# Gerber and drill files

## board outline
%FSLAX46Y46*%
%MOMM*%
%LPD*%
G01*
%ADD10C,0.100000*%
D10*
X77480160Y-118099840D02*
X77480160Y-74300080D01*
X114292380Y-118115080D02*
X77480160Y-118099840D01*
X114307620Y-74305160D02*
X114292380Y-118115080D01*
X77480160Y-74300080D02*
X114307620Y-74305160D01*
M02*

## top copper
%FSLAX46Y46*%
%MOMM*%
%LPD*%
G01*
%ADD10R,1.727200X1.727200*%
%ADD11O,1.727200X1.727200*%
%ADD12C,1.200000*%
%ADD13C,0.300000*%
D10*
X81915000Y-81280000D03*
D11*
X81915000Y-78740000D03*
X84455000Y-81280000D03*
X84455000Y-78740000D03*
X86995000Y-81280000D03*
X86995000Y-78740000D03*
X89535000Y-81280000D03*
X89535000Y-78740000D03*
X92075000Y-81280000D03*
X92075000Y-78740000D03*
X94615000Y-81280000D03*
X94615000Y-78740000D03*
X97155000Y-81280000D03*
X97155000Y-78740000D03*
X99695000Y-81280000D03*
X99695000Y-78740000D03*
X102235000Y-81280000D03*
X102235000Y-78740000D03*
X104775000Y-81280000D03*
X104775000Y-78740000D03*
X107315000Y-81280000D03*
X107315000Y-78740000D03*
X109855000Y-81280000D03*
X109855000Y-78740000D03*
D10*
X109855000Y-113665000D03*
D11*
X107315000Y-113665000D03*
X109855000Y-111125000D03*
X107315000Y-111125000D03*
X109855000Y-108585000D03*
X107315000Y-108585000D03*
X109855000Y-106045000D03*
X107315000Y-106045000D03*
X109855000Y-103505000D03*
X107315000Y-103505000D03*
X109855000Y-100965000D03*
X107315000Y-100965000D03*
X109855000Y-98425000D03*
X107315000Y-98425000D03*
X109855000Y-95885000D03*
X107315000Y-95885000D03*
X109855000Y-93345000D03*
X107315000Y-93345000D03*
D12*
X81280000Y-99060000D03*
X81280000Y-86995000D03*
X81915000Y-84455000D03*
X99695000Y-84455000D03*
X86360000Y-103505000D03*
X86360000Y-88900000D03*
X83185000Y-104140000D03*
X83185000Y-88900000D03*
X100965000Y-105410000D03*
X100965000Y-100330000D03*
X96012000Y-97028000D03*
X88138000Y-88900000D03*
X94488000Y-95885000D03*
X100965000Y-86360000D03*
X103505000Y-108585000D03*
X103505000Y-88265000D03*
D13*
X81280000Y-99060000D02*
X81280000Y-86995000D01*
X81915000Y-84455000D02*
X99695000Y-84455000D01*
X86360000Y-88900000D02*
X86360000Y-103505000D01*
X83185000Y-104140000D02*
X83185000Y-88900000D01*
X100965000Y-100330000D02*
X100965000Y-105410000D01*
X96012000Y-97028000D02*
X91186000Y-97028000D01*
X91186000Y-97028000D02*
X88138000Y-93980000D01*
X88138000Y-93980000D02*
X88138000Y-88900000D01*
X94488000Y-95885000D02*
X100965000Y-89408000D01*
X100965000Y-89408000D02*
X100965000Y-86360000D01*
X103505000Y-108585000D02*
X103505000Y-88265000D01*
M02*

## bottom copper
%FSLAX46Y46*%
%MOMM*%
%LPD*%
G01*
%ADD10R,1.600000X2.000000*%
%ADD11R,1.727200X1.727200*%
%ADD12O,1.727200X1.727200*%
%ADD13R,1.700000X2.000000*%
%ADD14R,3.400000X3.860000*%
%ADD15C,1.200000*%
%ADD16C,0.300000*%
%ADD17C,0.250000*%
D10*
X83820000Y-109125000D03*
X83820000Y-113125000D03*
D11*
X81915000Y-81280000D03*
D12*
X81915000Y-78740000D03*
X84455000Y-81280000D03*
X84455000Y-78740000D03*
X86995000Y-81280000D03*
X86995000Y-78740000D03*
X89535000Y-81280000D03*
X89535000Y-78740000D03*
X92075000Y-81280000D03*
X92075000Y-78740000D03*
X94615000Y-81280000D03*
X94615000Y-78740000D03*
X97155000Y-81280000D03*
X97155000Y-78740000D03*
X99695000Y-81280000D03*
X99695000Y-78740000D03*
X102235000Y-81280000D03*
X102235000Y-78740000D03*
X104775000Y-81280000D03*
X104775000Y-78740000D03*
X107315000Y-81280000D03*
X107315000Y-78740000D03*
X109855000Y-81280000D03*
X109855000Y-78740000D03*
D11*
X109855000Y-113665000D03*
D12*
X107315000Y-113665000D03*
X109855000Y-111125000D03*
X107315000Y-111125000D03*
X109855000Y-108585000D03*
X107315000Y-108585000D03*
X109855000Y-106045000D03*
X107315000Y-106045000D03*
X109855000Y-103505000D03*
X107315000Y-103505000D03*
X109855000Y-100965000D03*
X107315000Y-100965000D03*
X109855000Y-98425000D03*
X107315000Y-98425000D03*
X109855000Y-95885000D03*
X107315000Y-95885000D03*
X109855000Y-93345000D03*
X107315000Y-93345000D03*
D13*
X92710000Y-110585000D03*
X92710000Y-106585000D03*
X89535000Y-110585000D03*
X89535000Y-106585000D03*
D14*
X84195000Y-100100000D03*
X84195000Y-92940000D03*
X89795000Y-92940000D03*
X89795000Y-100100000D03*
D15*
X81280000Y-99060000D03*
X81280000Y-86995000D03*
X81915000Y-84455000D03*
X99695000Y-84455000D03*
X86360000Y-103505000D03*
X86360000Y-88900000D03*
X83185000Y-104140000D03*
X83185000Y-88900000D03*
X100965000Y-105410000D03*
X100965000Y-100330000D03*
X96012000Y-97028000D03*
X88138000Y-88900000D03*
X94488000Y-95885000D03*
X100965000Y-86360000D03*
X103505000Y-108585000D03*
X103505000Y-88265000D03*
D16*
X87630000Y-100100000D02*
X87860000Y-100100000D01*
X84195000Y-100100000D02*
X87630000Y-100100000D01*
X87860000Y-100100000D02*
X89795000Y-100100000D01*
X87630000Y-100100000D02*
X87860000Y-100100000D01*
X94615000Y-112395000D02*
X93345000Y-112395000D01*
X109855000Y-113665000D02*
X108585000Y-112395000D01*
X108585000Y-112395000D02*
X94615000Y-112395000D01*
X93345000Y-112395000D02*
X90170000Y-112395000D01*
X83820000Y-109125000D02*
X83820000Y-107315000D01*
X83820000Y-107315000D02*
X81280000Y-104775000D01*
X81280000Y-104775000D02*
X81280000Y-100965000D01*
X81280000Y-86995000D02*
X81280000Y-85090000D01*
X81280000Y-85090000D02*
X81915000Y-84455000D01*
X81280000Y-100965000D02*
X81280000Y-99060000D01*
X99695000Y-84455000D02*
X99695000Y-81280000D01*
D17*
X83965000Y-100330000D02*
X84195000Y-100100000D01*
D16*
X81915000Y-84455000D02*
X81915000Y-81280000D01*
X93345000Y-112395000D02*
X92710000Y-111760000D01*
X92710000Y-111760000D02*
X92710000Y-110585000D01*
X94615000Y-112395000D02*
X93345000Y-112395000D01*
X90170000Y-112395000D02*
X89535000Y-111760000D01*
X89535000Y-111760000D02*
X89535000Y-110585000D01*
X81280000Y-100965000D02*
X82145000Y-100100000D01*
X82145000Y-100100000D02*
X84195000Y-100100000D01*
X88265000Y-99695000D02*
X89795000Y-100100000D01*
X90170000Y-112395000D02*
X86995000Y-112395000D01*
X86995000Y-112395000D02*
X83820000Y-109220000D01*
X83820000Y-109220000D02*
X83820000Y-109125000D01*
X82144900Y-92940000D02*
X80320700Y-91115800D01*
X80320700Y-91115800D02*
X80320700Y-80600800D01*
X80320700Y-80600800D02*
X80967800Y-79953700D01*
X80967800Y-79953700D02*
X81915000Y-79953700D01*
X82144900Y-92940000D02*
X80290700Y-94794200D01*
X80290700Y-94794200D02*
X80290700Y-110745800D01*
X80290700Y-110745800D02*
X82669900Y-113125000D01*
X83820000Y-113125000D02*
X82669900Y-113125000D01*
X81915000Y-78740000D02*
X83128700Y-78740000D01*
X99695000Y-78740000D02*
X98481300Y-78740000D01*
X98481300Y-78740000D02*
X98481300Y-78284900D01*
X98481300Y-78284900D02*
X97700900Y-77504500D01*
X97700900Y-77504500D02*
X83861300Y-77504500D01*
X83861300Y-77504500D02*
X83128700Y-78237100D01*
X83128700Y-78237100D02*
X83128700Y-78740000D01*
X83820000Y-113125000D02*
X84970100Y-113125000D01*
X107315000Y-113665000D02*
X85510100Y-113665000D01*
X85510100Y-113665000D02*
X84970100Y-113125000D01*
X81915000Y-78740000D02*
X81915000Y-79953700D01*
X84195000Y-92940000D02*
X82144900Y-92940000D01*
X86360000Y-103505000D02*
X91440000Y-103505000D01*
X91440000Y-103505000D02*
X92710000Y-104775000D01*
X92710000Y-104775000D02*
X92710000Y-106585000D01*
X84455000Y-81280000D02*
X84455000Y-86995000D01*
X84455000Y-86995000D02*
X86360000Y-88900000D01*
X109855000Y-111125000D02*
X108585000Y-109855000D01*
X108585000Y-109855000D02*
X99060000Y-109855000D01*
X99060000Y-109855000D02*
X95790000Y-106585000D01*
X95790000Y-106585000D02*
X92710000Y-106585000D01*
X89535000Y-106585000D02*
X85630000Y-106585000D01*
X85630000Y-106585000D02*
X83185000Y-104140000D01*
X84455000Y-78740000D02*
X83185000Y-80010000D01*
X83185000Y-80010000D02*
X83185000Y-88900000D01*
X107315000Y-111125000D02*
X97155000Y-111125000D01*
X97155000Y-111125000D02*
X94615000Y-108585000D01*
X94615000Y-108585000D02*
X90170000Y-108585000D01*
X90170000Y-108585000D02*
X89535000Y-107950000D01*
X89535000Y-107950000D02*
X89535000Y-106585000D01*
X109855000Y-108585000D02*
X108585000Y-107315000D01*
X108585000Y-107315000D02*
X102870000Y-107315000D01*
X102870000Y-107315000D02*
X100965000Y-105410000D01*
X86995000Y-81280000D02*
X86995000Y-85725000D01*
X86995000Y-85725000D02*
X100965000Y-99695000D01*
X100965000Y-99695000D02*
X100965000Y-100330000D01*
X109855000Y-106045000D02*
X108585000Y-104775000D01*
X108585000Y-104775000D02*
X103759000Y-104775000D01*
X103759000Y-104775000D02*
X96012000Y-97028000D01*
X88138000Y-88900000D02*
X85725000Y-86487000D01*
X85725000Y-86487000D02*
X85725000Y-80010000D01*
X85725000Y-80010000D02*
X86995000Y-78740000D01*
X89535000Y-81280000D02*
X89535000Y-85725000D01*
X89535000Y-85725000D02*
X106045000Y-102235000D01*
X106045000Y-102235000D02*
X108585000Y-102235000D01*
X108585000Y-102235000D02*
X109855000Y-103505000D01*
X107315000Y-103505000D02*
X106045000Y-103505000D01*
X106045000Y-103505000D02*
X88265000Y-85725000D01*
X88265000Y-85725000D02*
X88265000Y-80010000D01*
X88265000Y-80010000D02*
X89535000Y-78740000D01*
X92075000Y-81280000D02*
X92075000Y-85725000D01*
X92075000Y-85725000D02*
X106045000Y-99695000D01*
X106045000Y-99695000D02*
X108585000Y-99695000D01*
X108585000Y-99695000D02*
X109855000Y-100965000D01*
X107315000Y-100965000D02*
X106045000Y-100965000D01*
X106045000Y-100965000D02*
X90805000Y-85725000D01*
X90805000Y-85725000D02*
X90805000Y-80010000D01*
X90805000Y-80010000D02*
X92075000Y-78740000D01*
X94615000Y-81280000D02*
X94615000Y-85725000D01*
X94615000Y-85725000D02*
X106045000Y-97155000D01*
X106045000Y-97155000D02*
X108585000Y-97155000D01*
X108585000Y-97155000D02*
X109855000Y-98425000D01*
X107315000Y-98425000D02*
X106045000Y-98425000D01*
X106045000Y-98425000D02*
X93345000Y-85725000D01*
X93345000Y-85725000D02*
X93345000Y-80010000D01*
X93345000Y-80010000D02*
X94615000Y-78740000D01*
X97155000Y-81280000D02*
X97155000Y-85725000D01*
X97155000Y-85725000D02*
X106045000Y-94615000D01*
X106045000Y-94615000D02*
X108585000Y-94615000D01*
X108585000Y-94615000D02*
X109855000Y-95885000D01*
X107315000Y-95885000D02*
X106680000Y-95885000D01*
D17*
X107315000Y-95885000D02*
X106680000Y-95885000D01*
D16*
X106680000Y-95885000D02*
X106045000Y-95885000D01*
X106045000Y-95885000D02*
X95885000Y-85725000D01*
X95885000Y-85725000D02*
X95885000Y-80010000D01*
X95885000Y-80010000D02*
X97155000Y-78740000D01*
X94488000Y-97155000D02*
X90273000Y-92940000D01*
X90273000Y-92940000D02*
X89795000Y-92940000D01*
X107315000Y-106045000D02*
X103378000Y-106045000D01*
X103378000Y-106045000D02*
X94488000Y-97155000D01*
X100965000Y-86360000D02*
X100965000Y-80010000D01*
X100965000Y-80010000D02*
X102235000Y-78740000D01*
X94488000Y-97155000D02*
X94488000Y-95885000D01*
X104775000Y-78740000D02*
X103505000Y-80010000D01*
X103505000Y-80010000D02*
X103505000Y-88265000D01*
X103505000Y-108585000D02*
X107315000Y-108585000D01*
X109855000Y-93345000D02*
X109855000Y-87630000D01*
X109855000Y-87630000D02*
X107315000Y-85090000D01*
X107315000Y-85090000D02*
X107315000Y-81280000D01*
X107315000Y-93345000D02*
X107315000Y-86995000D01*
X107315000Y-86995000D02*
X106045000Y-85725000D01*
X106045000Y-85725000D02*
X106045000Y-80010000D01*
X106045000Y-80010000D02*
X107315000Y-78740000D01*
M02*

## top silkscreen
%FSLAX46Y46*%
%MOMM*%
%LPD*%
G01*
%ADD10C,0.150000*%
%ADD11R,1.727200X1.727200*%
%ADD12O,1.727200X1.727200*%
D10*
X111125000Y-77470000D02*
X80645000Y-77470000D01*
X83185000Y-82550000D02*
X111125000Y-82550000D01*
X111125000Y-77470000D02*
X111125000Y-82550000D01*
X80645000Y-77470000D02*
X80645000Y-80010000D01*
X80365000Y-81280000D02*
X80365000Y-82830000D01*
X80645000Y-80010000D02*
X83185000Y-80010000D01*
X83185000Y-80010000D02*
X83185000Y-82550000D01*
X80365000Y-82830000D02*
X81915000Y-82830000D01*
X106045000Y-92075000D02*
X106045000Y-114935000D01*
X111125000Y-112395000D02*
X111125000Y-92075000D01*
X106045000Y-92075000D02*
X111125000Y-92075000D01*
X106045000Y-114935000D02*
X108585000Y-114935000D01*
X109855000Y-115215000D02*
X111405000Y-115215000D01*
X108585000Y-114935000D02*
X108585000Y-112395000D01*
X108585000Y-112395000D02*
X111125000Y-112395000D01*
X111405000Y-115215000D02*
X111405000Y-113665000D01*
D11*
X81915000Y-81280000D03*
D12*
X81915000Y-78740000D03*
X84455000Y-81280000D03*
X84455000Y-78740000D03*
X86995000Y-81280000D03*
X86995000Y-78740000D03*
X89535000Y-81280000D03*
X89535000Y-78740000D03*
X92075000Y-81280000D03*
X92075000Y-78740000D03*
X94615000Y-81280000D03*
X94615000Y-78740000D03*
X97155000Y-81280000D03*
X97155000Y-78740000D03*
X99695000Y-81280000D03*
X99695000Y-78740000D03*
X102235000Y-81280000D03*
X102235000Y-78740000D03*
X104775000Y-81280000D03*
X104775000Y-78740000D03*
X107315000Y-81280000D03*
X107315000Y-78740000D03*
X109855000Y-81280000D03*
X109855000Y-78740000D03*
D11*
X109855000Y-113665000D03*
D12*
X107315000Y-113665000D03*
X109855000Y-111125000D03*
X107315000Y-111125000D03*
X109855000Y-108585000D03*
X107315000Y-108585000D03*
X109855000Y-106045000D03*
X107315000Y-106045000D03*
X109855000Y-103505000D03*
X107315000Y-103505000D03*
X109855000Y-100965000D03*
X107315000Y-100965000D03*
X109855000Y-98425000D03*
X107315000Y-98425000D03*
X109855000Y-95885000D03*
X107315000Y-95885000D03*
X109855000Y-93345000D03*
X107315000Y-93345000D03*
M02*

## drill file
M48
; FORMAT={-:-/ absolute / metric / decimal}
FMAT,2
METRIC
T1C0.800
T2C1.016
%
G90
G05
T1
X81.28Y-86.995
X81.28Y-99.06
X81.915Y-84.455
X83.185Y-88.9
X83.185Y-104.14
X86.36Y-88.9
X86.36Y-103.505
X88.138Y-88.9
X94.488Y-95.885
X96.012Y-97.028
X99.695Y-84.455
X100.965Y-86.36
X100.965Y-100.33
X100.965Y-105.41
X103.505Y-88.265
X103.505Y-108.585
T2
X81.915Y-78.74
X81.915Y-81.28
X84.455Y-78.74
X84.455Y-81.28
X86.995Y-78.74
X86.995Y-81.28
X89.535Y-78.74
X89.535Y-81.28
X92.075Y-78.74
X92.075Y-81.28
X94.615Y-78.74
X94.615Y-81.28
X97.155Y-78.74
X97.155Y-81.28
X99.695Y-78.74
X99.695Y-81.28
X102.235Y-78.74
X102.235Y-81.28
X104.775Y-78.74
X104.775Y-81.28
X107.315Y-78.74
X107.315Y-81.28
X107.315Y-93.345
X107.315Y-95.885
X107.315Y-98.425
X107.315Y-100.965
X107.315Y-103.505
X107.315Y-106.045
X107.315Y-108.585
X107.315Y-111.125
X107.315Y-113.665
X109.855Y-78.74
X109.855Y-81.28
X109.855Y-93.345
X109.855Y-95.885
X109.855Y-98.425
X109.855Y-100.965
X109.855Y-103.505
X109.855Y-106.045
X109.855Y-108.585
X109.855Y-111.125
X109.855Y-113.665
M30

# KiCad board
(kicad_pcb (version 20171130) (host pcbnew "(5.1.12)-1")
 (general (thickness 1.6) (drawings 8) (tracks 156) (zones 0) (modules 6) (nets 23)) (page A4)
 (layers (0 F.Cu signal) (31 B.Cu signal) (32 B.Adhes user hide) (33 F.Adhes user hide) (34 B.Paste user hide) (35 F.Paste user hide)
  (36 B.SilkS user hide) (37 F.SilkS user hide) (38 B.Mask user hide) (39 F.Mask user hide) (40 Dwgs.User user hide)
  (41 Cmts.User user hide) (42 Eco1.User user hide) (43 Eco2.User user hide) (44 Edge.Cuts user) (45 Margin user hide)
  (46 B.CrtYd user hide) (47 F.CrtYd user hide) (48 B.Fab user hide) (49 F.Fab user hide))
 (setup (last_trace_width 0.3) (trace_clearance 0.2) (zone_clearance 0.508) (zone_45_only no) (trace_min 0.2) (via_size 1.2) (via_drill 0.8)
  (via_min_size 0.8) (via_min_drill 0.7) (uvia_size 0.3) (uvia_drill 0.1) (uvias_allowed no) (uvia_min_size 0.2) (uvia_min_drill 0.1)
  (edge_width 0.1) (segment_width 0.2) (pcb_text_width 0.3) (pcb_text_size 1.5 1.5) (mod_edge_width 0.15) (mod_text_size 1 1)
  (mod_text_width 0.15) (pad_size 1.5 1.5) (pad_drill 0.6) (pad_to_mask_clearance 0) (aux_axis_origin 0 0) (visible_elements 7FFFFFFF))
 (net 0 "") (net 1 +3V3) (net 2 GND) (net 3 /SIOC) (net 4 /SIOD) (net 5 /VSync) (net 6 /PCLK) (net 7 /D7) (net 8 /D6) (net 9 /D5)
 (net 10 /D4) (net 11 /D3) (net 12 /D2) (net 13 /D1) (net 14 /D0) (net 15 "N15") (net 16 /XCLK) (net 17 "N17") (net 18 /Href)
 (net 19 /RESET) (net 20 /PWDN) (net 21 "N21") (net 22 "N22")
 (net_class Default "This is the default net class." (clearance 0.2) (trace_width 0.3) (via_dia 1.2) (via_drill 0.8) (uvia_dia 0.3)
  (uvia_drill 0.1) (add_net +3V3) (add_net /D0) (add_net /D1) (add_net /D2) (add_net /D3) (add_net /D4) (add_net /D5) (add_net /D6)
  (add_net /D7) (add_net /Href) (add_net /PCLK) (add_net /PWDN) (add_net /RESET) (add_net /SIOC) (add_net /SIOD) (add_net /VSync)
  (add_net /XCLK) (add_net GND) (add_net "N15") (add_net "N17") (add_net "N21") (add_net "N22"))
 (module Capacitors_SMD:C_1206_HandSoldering (layer B.Cu) (at 83.82 111.125 270)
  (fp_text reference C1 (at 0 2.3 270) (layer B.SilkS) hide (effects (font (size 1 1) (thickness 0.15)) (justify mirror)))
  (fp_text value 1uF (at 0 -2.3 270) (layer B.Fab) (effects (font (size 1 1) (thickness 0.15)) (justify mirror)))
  (pad 1 smd rect (at -2 0 270) (size 2 1.6) (layers B.Cu B.Paste B.Mask) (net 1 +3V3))
  (pad 2 smd rect (at 2 0 270) (size 2 1.6) (layers B.Cu B.Paste B.Mask) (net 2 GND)))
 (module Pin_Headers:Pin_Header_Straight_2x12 (layer F.Cu) (at 81.915 81.28 90)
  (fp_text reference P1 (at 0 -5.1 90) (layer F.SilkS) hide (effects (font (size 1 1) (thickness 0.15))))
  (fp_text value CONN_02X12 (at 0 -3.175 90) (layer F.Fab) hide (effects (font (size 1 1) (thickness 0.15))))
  (fp_line (start 3.81 29.21) (end 3.81 -1.27) (layer F.SilkS) (width 0.15))
  (fp_line (start -1.27 1.27) (end -1.27 29.21) (layer F.SilkS) (width 0.15))
  (fp_line (start 3.81 29.21) (end -1.27 29.21) (layer F.SilkS) (width 0.15))
  (fp_line (start 3.81 -1.27) (end 1.27 -1.27) (layer F.SilkS) (width 0.15))
  (fp_line (start 0 -1.55) (end -1.55 -1.55) (layer F.SilkS) (width 0.15))
  (fp_line (start 1.27 -1.27) (end 1.27 1.27) (layer F.SilkS) (width 0.15))
  (fp_line (start 1.27 1.27) (end -1.27 1.27) (layer F.SilkS) (width 0.15))
  (fp_line (start -1.55 -1.55) (end -1.55 0) (layer F.SilkS) (width 0.15))
  (pad 1 thru_hole rect (at 0 0 90) (size 1.7272 1.7272) (drill 1.016) (layers *.Cu *.Mask F.SilkS) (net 1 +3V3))
  (pad 2 thru_hole oval (at 2.54 0 90) (size 1.7272 1.7272) (drill 1.016) (layers *.Cu *.Mask F.SilkS) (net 2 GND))
  (pad 3 thru_hole oval (at 0 2.54 90) (size 1.7272 1.7272) (drill 1.016) (layers *.Cu *.Mask F.SilkS) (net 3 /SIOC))
  (pad 4 thru_hole oval (at 2.54 2.54 90) (size 1.7272 1.7272) (drill 1.016) (layers *.Cu *.Mask F.SilkS) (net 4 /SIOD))
  (pad 5 thru_hole oval (at 0 5.08 90) (size 1.7272 1.7272) (drill 1.016) (layers *.Cu *.Mask F.SilkS) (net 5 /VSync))
  (pad 6 thru_hole oval (at 2.54 5.08 90) (size 1.7272 1.7272) (drill 1.016) (layers *.Cu *.Mask F.SilkS) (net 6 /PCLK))
  (pad 7 thru_hole oval (at 0 7.62 90) (size 1.7272 1.7272) (drill 1.016) (layers *.Cu *.Mask F.SilkS) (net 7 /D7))
  (pad 8 thru_hole oval (at 2.54 7.62 90) (size 1.7272 1.7272) (drill 1.016) (layers *.Cu *.Mask F.SilkS) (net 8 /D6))
  (pad 9 thru_hole oval (at 0 10.16 90) (size 1.7272 1.7272) (drill 1.016) (layers *.Cu *.Mask F.SilkS) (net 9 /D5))
  (pad 10 thru_hole oval (at 2.54 10.16 90) (size 1.7272 1.7272) (drill 1.016) (layers *.Cu *.Mask F.SilkS) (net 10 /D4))
  (pad 11 thru_hole oval (at 0 12.7 90) (size 1.7272 1.7272) (drill 1.016) (layers *.Cu *.Mask F.SilkS) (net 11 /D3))
  (pad 12 thru_hole oval (at 2.54 12.7 90) (size 1.7272 1.7272) (drill 1.016) (layers *.Cu *.Mask F.SilkS) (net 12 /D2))
  (pad 13 thru_hole oval (at 0 15.24 90) (size 1.7272 1.7272) (drill 1.016) (layers *.Cu *.Mask F.SilkS) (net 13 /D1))
  (pad 14 thru_hole oval (at 2.54 15.24 90) (size 1.7272 1.7272) (drill 1.016) (layers *.Cu *.Mask F.SilkS) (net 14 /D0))
  (pad 15 thru_hole oval (at 0 17.78 90) (size 1.7272 1.7272) (drill 1.016) (layers *.Cu *.Mask F.SilkS) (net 1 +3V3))
  (pad 16 thru_hole oval (at 2.54 17.78 90) (size 1.7272 1.7272) (drill 1.016) (layers *.Cu *.Mask F.SilkS) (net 2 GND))
  (pad 17 thru_hole oval (at 0 20.32 90) (size 1.7272 1.7272) (drill 1.016) (layers *.Cu *.Mask F.SilkS) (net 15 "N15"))
  (pad 18 thru_hole oval (at 2.54 20.32 90) (size 1.7272 1.7272) (drill 1.016) (layers *.Cu *.Mask F.SilkS) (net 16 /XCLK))
  (pad 19 thru_hole oval (at 0 22.86 90) (size 1.7272 1.7272) (drill 1.016) (layers *.Cu *.Mask F.SilkS) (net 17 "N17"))
  (pad 20 thru_hole oval (at 2.54 22.86 90) (size 1.7272 1.7272) (drill 1.016) (layers *.Cu *.Mask F.SilkS) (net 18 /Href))
  (pad 21 thru_hole oval (at 0 25.4 90) (size 1.7272 1.7272) (drill 1.016) (layers *.Cu *.Mask F.SilkS) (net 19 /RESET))
  (pad 22 thru_hole oval (at 2.54 25.4 90) (size 1.7272 1.7272) (drill 1.016) (layers *.Cu *.Mask F.SilkS) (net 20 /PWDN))
  (pad 23 thru_hole oval (at 0 27.94 90) (size 1.7272 1.7272) (drill 1.016) (layers *.Cu *.Mask F.SilkS) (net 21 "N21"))
  (pad 24 thru_hole oval (at 2.54 27.94 90) (size 1.7272 1.7272) (drill 1.016) (layers *.Cu *.Mask F.SilkS) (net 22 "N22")))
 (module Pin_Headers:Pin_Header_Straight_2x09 (layer F.Cu) (at 109.855 113.665 180)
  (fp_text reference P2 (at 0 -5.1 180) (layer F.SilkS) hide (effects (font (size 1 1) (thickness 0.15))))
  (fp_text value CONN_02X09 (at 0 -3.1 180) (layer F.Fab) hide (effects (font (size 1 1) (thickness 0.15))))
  (fp_line (start 3.81 21.59) (end 3.81 -1.27) (layer F.SilkS) (width 0.15))
  (fp_line (start -1.27 1.27) (end -1.27 21.59) (layer F.SilkS) (width 0.15))
  (fp_line (start 3.81 21.59) (end -1.27 21.59) (layer F.SilkS) (width 0.15))
  (fp_line (start 3.81 -1.27) (end 1.27 -1.27) (layer F.SilkS) (width 0.15))
  (fp_line (start 0 -1.55) (end -1.55 -1.55) (layer F.SilkS) (width 0.15))
  (fp_line (start 1.27 -1.27) (end 1.27 1.27) (layer F.SilkS) (width 0.15))
  (fp_line (start 1.27 1.27) (end -1.27 1.27) (layer F.SilkS) (width 0.15))
  (fp_line (start -1.55 -1.55) (end -1.55 0) (layer F.SilkS) (width 0.15))
  (pad 1 thru_hole rect (at 0 0 180) (size 1.7272 1.7272) (drill 1.016) (layers *.Cu *.Mask F.SilkS) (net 1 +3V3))
  (pad 2 thru_hole oval (at 2.54 0 180) (size 1.7272 1.7272) (drill 1.016) (layers *.Cu *.Mask F.SilkS) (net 2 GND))
  (pad 3 thru_hole oval (at 0 2.54 180) (size 1.7272 1.7272) (drill 1.016) (layers *.Cu *.Mask F.SilkS) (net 3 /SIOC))
  (pad 4 thru_hole oval (at 2.54 2.54 180) (size 1.7272 1.7272) (drill 1.016) (layers *.Cu *.Mask F.SilkS) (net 4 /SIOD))
  (pad 5 thru_hole oval (at 0 5.08 180) (size 1.7272 1.7272) (drill 1.016) (layers *.Cu *.Mask F.SilkS) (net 5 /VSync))
  (pad 6 thru_hole oval (at 2.54 5.08 180) (size 1.7272 1.7272) (drill 1.016) (layers *.Cu *.Mask F.SilkS) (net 18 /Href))
  (pad 7 thru_hole oval (at 0 7.62 180) (size 1.7272 1.7272) (drill 1.016) (layers *.Cu *.Mask F.SilkS) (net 6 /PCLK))
  (pad 8 thru_hole oval (at 2.54 7.62 180) (size 1.7272 1.7272) (drill 1.016) (layers *.Cu *.Mask F.SilkS) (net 16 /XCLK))
  (pad 9 thru_hole oval (at 0 10.16 180) (size 1.7272 1.7272) (drill 1.016) (layers *.Cu *.Mask F.SilkS) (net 7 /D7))
  (pad 10 thru_hole oval (at 2.54 10.16 180) (size 1.7272 1.7272) (drill 1.016) (layers *.Cu *.Mask F.SilkS) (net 8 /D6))
  (pad 11 thru_hole oval (at 0 12.7 180) (size 1.7272 1.7272) (drill 1.016) (layers *.Cu *.Mask F.SilkS) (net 9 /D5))
  (pad 12 thru_hole oval (at 2.54 12.7 180) (size 1.7272 1.7272) (drill 1.016) (layers *.Cu *.Mask F.SilkS) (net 10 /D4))
  (pad 13 thru_hole oval (at 0 15.24 180) (size 1.7272 1.7272) (drill 1.016) (layers *.Cu *.Mask F.SilkS) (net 11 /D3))
  (pad 14 thru_hole oval (at 2.54 15.24 180) (size 1.7272 1.7272) (drill 1.016) (layers *.Cu *.Mask F.SilkS) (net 12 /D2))
  (pad 15 thru_hole oval (at 0 17.78 180) (size 1.7272 1.7272) (drill 1.016) (layers *.Cu *.Mask F.SilkS) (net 13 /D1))
  (pad 16 thru_hole oval (at 2.54 17.78 180) (size 1.7272 1.7272) (drill 1.016) (layers *.Cu *.Mask F.SilkS) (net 14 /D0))
  (pad 17 thru_hole oval (at 0 20.32 180) (size 1.7272 1.7272) (drill 1.016) (layers *.Cu *.Mask F.SilkS) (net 19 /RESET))
  (pad 18 thru_hole oval (at 2.54 20.32 180) (size 1.7272 1.7272) (drill 1.016) (layers *.Cu *.Mask F.SilkS) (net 20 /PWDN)))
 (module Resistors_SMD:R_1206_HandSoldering (layer B.Cu) (at 92.71 108.585 90)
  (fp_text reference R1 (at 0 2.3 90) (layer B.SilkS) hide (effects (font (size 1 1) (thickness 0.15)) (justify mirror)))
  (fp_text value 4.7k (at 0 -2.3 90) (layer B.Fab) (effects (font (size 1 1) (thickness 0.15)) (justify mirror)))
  (pad 1 smd rect (at -2 0 90) (size 2 1.7) (layers B.Cu B.Paste B.Mask) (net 1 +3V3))
  (pad 2 smd rect (at 2 0 90) (size 2 1.7) (layers B.Cu B.Paste B.Mask) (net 3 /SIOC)))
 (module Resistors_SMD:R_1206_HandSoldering (layer B.Cu) (at 89.535 108.585 90)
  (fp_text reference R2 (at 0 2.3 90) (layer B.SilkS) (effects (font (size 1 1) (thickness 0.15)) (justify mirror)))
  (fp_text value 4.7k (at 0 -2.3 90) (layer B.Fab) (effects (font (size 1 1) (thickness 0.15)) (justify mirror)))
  (pad 1 smd rect (at -2 0 90) (size 2 1.7) (layers B.Cu B.Paste B.Mask) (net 1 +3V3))
  (pad 2 smd rect (at 2 0 90) (size 2 1.7) (layers B.Cu B.Paste B.Mask) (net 4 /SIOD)))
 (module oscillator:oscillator (layer B.Cu) (at 86.995 96.52 90)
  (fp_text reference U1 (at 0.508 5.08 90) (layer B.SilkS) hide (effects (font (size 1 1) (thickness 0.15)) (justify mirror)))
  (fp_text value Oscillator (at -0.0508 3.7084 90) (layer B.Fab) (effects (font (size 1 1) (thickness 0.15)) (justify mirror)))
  (pad 1 smd rect (at -3.58 -2.8 90) (size 3.86 3.4) (layers B.Cu B.Paste B.Mask) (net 1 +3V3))
  (pad 2 smd rect (at 3.58 -2.8 90) (size 3.86 3.4) (layers B.Cu B.Paste B.Mask) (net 2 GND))
  (pad 3 smd rect (at 3.58 2.8 90) (size 3.86 3.4) (layers B.Cu B.Paste B.Mask) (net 16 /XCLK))
  (pad 4 smd rect (at -3.58 2.8 90) (size 3.86 3.4) (layers B.Cu B.Paste B.Mask) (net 1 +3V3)))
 (gr_line (start 77.48016 118.09984) (end 77.48016 74.30008) (layer Edge.Cuts) (width 0.1))
 (gr_line (start 114.29238 118.11508) (end 77.48016 118.09984) (layer Edge.Cuts) (width 0.1))
 (gr_line (start 114.30762 74.30516) (end 114.29238 118.11508) (layer Edge.Cuts) (width 0.1))
 (gr_line (start 77.48016 74.30008) (end 114.30762 74.30516) (layer Edge.Cuts) (width 0.1))
 (segment (start 87.63 100.1) (end 87.86 100.1) (width 0.3) (layer B.Cu) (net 1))
 (segment (start 84.195 100.1) (end 87.63 100.1) (width 0.3) (layer B.Cu) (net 1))
 (segment (start 87.86 100.1) (end 89.795 100.1) (width 0.3) (layer B.Cu) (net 1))
 (segment (start 87.63 100.1) (end 87.86 100.1) (width 0.3) (layer B.Cu) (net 1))
 (segment (start 94.615 112.395) (end 93.345 112.395) (width 0.3) (layer B.Cu) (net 1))
 (segment (start 109.855 113.665) (end 108.585 112.395) (width 0.3) (layer B.Cu) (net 1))
 (segment (start 108.585 112.395) (end 94.615 112.395) (width 0.3) (layer B.Cu) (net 1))
 (segment (start 93.345 112.395) (end 90.17 112.395) (width 0.3) (layer B.Cu) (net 1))
 (segment (start 83.82 109.125) (end 83.82 107.315) (width 0.3) (layer B.Cu) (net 1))
 (segment (start 83.82 107.315) (end 81.28 104.775) (width 0.3) (layer B.Cu) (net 1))
 (segment (start 81.28 104.775) (end 81.28 100.965) (width 0.3) (layer B.Cu) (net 1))
 (segment (start 81.28 99.06) (end 81.28 86.995) (width 0.3) (layer F.Cu) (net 1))
 (segment (start 81.28 86.995) (end 81.28 85.09) (width 0.3) (layer B.Cu) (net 1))
 (segment (start 81.28 85.09) (end 81.915 84.455) (width 0.3) (layer B.Cu) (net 1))
 (segment (start 81.28 100.965) (end 81.28 99.06) (width 0.3) (layer B.Cu) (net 1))
 (segment (start 99.695 84.455) (end 99.695 81.28) (width 0.3) (layer B.Cu) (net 1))
 (segment (start 81.915 84.455) (end 99.695 84.455) (width 0.3) (layer F.Cu) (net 1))
 (segment (start 83.965 100.33) (end 84.195 100.1) (width 0.25) (layer B.Cu) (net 1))
 (segment (start 81.915 84.455) (end 81.915 81.28) (width 0.3) (layer B.Cu) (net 1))
 (segment (start 93.345 112.395) (end 92.71 111.76) (width 0.3) (layer B.Cu) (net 1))
 (segment (start 92.71 111.76) (end 92.71 110.585) (width 0.3) (layer B.Cu) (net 1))
 (segment (start 94.615 112.395) (end 93.345 112.395) (width 0.3) (layer B.Cu) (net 1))
 (segment (start 90.17 112.395) (end 89.535 111.76) (width 0.3) (layer B.Cu) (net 1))
 (segment (start 89.535 111.76) (end 89.535 110.585) (width 0.3) (layer B.Cu) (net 1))
 (segment (start 81.28 100.965) (end 82.145 100.1) (width 0.3) (layer B.Cu) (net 1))
 (segment (start 82.145 100.1) (end 84.195 100.1) (width 0.3) (layer B.Cu) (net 1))
 (segment (start 88.265 99.695) (end 89.795 100.1) (width 0.3) (layer B.Cu) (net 1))
 (segment (start 90.17 112.395) (end 86.995 112.395) (width 0.3) (layer B.Cu) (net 1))
 (segment (start 86.995 112.395) (end 83.82 109.22) (width 0.3) (layer B.Cu) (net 1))
 (segment (start 83.82 109.22) (end 83.82 109.125) (width 0.3) (layer B.Cu) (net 1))
 (via (at 81.28 99.06) (size 1.2) (layers F.Cu B.Cu) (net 1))
 (via (at 81.28 86.995) (size 1.2) (layers F.Cu B.Cu) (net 1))
 (via (at 81.915 84.455) (size 1.2) (layers F.Cu B.Cu) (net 1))
 (via (at 99.695 84.455) (size 1.2) (layers F.Cu B.Cu) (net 1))
 (segment (start 82.1449 92.94) (end 80.3207 91.1158) (width 0.3) (layer B.Cu) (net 2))
 (segment (start 80.3207 91.1158) (end 80.3207 80.6008) (width 0.3) (layer B.Cu) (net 2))
 (segment (start 80.3207 80.6008) (end 80.9678 79.9537) (width 0.3) (layer B.Cu) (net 2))
 (segment (start 80.9678 79.9537) (end 81.915 79.9537) (width 0.3) (layer B.Cu) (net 2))
 (segment (start 82.1449 92.94) (end 80.2907 94.7942) (width 0.3) (layer B.Cu) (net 2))
 (segment (start 80.2907 94.7942) (end 80.2907 110.7458) (width 0.3) (layer B.Cu) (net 2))
 (segment (start 80.2907 110.7458) (end 82.6699 113.125) (width 0.3) (layer B.Cu) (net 2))
 (segment (start 83.82 113.125) (end 82.6699 113.125) (width 0.3) (layer B.Cu) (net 2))
 (segment (start 81.915 78.74) (end 83.1287 78.74) (width 0.3) (layer B.Cu) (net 2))
 (segment (start 99.695 78.74) (end 98.4813 78.74) (width 0.3) (layer B.Cu) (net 2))
 (segment (start 98.4813 78.74) (end 98.4813 78.2849) (width 0.3) (layer B.Cu) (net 2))
 (segment (start 98.4813 78.2849) (end 97.7009 77.5045) (width 0.3) (layer B.Cu) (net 2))
 (segment (start 97.7009 77.5045) (end 83.8613 77.5045) (width 0.3) (layer B.Cu) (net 2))
 (segment (start 83.8613 77.5045) (end 83.1287 78.2371) (width 0.3) (layer B.Cu) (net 2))
 (segment (start 83.1287 78.2371) (end 83.1287 78.74) (width 0.3) (layer B.Cu) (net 2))
 (segment (start 83.82 113.125) (end 84.9701 113.125) (width 0.3) (layer B.Cu) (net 2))
 (segment (start 107.315 113.665) (end 85.5101 113.665) (width 0.3) (layer B.Cu) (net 2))
 (segment (start 85.5101 113.665) (end 84.9701 113.125) (width 0.3) (layer B.Cu) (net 2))
 (segment (start 81.915 78.74) (end 81.915 79.9537) (width 0.3) (layer B.Cu) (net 2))
 (segment (start 84.195 92.94) (end 82.1449 92.94) (width 0.3) (layer B.Cu) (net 2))
 (segment (start 86.36 103.505) (end 91.44 103.505) (width 0.3) (layer B.Cu) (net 3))
 (segment (start 91.44 103.505) (end 92.71 104.775) (width 0.3) (layer B.Cu) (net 3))
 (segment (start 92.71 104.775) (end 92.71 106.585) (width 0.3) (layer B.Cu) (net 3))
 (segment (start 84.455 81.28) (end 84.455 86.995) (width 0.3) (layer B.Cu) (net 3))
 (segment (start 84.455 86.995) (end 86.36 88.9) (width 0.3) (layer B.Cu) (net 3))
 (segment (start 86.36 88.9) (end 86.36 103.505) (width 0.3) (layer F.Cu) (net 3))
 (segment (start 109.855 111.125) (end 108.585 109.855) (width 0.3) (layer B.Cu) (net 3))
 (segment (start 108.585 109.855) (end 99.06 109.855) (width 0.3) (layer B.Cu) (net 3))
 (segment (start 99.06 109.855) (end 95.79 106.585) (width 0.3) (layer B.Cu) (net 3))
 (segment (start 95.79 106.585) (end 92.71 106.585) (width 0.3) (layer B.Cu) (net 3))
 (via (at 86.36 103.505) (size 1.2) (layers F.Cu B.Cu) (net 3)) (via (at 86.36 88.9) (size 1.2) (layers F.Cu B.Cu) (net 3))
 (segment (start 89.535 106.585) (end 85.63 106.585) (width 0.3) (layer B.Cu) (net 4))
 (segment (start 85.63 106.585) (end 83.185 104.14) (width 0.3) (layer B.Cu) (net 4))
 (segment (start 83.185 104.14) (end 83.185 88.9) (width 0.3) (layer F.Cu) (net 4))
 (segment (start 84.455 78.74) (end 83.185 80.01) (width 0.3) (layer B.Cu) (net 4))
 (segment (start 83.185 80.01) (end 83.185 88.9) (width 0.3) (layer B.Cu) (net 4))
 (segment (start 107.315 111.125) (end 97.155 111.125) (width 0.3) (layer B.Cu) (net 4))
 (segment (start 97.155 111.125) (end 94.615 108.585) (width 0.3) (layer B.Cu) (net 4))
 (segment (start 94.615 108.585) (end 90.17 108.585) (width 0.3) (layer B.Cu) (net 4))
 (segment (start 90.17 108.585) (end 89.535 107.95) (width 0.3) (layer B.Cu) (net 4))
 (segment (start 89.535 107.95) (end 89.535 106.585) (width 0.3) (layer B.Cu) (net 4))
 (via (at 83.185 104.14) (size 1.2) (layers F.Cu B.Cu) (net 4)) (via (at 83.185 88.9) (size 1.2) (layers F.Cu B.Cu) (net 4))
 (segment (start 109.855 108.585) (end 108.585 107.315) (width 0.3) (layer B.Cu) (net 5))
 (segment (start 108.585 107.315) (end 102.87 107.315) (width 0.3) (layer B.Cu) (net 5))
 (segment (start 102.87 107.315) (end 100.965 105.41) (width 0.3) (layer B.Cu) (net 5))
 (segment (start 86.995 81.28) (end 86.995 85.725) (width 0.3) (layer B.Cu) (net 5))
 (segment (start 86.995 85.725) (end 100.965 99.695) (width 0.3) (layer B.Cu) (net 5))
 (segment (start 100.965 99.695) (end 100.965 100.33) (width 0.3) (layer B.Cu) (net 5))
 (segment (start 100.965 100.33) (end 100.965 105.41) (width 0.3) (layer F.Cu) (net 5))
 (via (at 100.965 105.41) (size 1.2) (layers F.Cu B.Cu) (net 5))
 (via (at 100.965 100.33) (size 1.2) (layers F.Cu B.Cu) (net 5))
 (segment (start 109.855 106.045) (end 108.585 104.775) (width 0.3) (layer B.Cu) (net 6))
 (segment (start 108.585 104.775) (end 103.759 104.775) (width 0.3) (layer B.Cu) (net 6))
 (segment (start 103.759 104.775) (end 96.012 97.028) (width 0.3) (layer B.Cu) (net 6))
 (segment (start 96.012 97.028) (end 91.186 97.028) (width 0.3) (layer F.Cu) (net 6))
 (segment (start 91.186 97.028) (end 88.138 93.98) (width 0.3) (layer F.Cu) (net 6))
 (segment (start 88.138 93.98) (end 88.138 88.9) (width 0.3) (layer F.Cu) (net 6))
 (segment (start 88.138 88.9) (end 85.725 86.487) (width 0.3) (layer B.Cu) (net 6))
 (segment (start 85.725 86.487) (end 85.725 80.01) (width 0.3) (layer B.Cu) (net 6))
 (segment (start 85.725 80.01) (end 86.995 78.74) (width 0.3) (layer B.Cu) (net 6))
 (via (at 96.012 97.028) (size 1.2) (layers F.Cu B.Cu) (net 6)) (via (at 88.138 88.9) (size 1.2) (layers F.Cu B.Cu) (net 6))
 (segment (start 89.535 81.28) (end 89.535 85.725) (width 0.3) (layer B.Cu) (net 7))
 (segment (start 89.535 85.725) (end 106.045 102.235) (width 0.3) (layer B.Cu) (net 7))
 (segment (start 106.045 102.235) (end 108.585 102.235) (width 0.3) (layer B.Cu) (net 7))
 (segment (start 108.585 102.235) (end 109.855 103.505) (width 0.3) (layer B.Cu) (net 7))
 (segment (start 107.315 103.505) (end 106.045 103.505) (width 0.3) (layer B.Cu) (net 8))
 (segment (start 106.045 103.505) (end 88.265 85.725) (width 0.3) (layer B.Cu) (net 8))
 (segment (start 88.265 85.725) (end 88.265 80.01) (width 0.3) (layer B.Cu) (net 8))
 (segment (start 88.265 80.01) (end 89.535 78.74) (width 0.3) (layer B.Cu) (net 8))
 (segment (start 92.075 81.28) (end 92.075 85.725) (width 0.3) (layer B.Cu) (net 9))
 (segment (start 92.075 85.725) (end 106.045 99.695) (width 0.3) (layer B.Cu) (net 9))
 (segment (start 106.045 99.695) (end 108.585 99.695) (width 0.3) (layer B.Cu) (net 9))
 (segment (start 108.585 99.695) (end 109.855 100.965) (width 0.3) (layer B.Cu) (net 9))
 (segment (start 107.315 100.965) (end 106.045 100.965) (width 0.3) (layer B.Cu) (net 10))
 (segment (start 106.045 100.965) (end 90.805 85.725) (width 0.3) (layer B.Cu) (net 10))
 (segment (start 90.805 85.725) (end 90.805 80.01) (width 0.3) (layer B.Cu) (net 10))
 (segment (start 90.805 80.01) (end 92.075 78.74) (width 0.3) (layer B.Cu) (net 10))
 (segment (start 94.615 81.28) (end 94.615 85.725) (width 0.3) (layer B.Cu) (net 11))
 (segment (start 94.615 85.725) (end 106.045 97.155) (width 0.3) (layer B.Cu) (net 11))
 (segment (start 106.045 97.155) (end 108.585 97.155) (width 0.3) (layer B.Cu) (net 11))
 (segment (start 108.585 97.155) (end 109.855 98.425) (width 0.3) (layer B.Cu) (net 11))
 (segment (start 107.315 98.425) (end 106.045 98.425) (width 0.3) (layer B.Cu) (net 12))
 (segment (start 106.045 98.425) (end 93.345 85.725) (width 0.3) (layer B.Cu) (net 12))
 (segment (start 93.345 85.725) (end 93.345 80.01) (width 0.3) (layer B.Cu) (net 12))
 (segment (start 93.345 80.01) (end 94.615 78.74) (width 0.3) (layer B.Cu) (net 12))
 (segment (start 97.155 81.28) (end 97.155 85.725) (width 0.3) (layer B.Cu) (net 13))
 (segment (start 97.155 85.725) (end 106.045 94.615) (width 0.3) (layer B.Cu) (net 13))
 (segment (start 106.045 94.615) (end 108.585 94.615) (width 0.3) (layer B.Cu) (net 13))
 (segment (start 108.585 94.615) (end 109.855 95.885) (width 0.3) (layer B.Cu) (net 13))
 (segment (start 107.315 95.885) (end 106.68 95.885) (width 0.3) (layer B.Cu) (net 14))
 (segment (start 107.315 95.885) (end 106.68 95.885) (width 0.25) (layer B.Cu) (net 14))
 (segment (start 106.68 95.885) (end 106.045 95.885) (width 0.3) (layer B.Cu) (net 14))
 (segment (start 106.045 95.885) (end 95.885 85.725) (width 0.3) (layer B.Cu) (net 14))
 (segment (start 95.885 85.725) (end 95.885 80.01) (width 0.3) (layer B.Cu) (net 14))
 (segment (start 95.885 80.01) (end 97.155 78.74) (width 0.3) (layer B.Cu) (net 14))
 (segment (start 94.488 97.155) (end 90.273 92.94) (width 0.3) (layer B.Cu) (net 16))
 (segment (start 90.273 92.94) (end 89.795 92.94) (width 0.3) (layer B.Cu) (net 16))
 (segment (start 107.315 106.045) (end 103.378 106.045) (width 0.3) (layer B.Cu) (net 16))
 (segment (start 103.378 106.045) (end 94.488 97.155) (width 0.3) (layer B.Cu) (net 16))
 (segment (start 94.488 95.885) (end 100.965 89.408) (width 0.3) (layer F.Cu) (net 16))
 (segment (start 100.965 89.408) (end 100.965 86.36) (width 0.3) (layer F.Cu) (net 16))
 (segment (start 100.965 86.36) (end 100.965 80.01) (width 0.3) (layer B.Cu) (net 16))
 (segment (start 100.965 80.01) (end 102.235 78.74) (width 0.3) (layer B.Cu) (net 16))
 (segment (start 94.488 97.155) (end 94.488 95.885) (width 0.3) (layer B.Cu) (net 16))
 (via (at 94.488 95.885) (size 1.2) (layers F.Cu B.Cu) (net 16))
 (via (at 100.965 86.36) (size 1.2) (layers F.Cu B.Cu) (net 16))
 (segment (start 103.505 108.585) (end 103.505 88.265) (width 0.3) (layer F.Cu) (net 18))
 (segment (start 104.775 78.74) (end 103.505 80.01) (width 0.3) (layer B.Cu) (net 18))
 (segment (start 103.505 80.01) (end 103.505 88.265) (width 0.3) (layer B.Cu) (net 18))
 (segment (start 103.505 108.585) (end 107.315 108.585) (width 0.3) (layer B.Cu) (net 18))
 (via (at 103.505 108.585) (size 1.2) (layers F.Cu B.Cu) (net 18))
 (via (at 103.505 88.265) (size 1.2) (layers F.Cu B.Cu) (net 18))
 (segment (start 109.855 93.345) (end 109.855 87.63) (width 0.3) (layer B.Cu) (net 19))
 (segment (start 109.855 87.63) (end 107.315 85.09) (width 0.3) (layer B.Cu) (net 19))
 (segment (start 107.315 85.09) (end 107.315 81.28) (width 0.3) (layer B.Cu) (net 19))
 (segment (start 107.315 93.345) (end 107.315 86.995) (width 0.3) (layer B.Cu) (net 20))
 (segment (start 107.315 86.995) (end 106.045 85.725) (width 0.3) (layer B.Cu) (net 20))
 (segment (start 106.045 85.725) (end 106.045 80.01) (width 0.3) (layer B.Cu) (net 20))
 (segment (start 106.045 80.01) (end 107.315 78.74) (width 0.3) (layer B.Cu) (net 20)))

